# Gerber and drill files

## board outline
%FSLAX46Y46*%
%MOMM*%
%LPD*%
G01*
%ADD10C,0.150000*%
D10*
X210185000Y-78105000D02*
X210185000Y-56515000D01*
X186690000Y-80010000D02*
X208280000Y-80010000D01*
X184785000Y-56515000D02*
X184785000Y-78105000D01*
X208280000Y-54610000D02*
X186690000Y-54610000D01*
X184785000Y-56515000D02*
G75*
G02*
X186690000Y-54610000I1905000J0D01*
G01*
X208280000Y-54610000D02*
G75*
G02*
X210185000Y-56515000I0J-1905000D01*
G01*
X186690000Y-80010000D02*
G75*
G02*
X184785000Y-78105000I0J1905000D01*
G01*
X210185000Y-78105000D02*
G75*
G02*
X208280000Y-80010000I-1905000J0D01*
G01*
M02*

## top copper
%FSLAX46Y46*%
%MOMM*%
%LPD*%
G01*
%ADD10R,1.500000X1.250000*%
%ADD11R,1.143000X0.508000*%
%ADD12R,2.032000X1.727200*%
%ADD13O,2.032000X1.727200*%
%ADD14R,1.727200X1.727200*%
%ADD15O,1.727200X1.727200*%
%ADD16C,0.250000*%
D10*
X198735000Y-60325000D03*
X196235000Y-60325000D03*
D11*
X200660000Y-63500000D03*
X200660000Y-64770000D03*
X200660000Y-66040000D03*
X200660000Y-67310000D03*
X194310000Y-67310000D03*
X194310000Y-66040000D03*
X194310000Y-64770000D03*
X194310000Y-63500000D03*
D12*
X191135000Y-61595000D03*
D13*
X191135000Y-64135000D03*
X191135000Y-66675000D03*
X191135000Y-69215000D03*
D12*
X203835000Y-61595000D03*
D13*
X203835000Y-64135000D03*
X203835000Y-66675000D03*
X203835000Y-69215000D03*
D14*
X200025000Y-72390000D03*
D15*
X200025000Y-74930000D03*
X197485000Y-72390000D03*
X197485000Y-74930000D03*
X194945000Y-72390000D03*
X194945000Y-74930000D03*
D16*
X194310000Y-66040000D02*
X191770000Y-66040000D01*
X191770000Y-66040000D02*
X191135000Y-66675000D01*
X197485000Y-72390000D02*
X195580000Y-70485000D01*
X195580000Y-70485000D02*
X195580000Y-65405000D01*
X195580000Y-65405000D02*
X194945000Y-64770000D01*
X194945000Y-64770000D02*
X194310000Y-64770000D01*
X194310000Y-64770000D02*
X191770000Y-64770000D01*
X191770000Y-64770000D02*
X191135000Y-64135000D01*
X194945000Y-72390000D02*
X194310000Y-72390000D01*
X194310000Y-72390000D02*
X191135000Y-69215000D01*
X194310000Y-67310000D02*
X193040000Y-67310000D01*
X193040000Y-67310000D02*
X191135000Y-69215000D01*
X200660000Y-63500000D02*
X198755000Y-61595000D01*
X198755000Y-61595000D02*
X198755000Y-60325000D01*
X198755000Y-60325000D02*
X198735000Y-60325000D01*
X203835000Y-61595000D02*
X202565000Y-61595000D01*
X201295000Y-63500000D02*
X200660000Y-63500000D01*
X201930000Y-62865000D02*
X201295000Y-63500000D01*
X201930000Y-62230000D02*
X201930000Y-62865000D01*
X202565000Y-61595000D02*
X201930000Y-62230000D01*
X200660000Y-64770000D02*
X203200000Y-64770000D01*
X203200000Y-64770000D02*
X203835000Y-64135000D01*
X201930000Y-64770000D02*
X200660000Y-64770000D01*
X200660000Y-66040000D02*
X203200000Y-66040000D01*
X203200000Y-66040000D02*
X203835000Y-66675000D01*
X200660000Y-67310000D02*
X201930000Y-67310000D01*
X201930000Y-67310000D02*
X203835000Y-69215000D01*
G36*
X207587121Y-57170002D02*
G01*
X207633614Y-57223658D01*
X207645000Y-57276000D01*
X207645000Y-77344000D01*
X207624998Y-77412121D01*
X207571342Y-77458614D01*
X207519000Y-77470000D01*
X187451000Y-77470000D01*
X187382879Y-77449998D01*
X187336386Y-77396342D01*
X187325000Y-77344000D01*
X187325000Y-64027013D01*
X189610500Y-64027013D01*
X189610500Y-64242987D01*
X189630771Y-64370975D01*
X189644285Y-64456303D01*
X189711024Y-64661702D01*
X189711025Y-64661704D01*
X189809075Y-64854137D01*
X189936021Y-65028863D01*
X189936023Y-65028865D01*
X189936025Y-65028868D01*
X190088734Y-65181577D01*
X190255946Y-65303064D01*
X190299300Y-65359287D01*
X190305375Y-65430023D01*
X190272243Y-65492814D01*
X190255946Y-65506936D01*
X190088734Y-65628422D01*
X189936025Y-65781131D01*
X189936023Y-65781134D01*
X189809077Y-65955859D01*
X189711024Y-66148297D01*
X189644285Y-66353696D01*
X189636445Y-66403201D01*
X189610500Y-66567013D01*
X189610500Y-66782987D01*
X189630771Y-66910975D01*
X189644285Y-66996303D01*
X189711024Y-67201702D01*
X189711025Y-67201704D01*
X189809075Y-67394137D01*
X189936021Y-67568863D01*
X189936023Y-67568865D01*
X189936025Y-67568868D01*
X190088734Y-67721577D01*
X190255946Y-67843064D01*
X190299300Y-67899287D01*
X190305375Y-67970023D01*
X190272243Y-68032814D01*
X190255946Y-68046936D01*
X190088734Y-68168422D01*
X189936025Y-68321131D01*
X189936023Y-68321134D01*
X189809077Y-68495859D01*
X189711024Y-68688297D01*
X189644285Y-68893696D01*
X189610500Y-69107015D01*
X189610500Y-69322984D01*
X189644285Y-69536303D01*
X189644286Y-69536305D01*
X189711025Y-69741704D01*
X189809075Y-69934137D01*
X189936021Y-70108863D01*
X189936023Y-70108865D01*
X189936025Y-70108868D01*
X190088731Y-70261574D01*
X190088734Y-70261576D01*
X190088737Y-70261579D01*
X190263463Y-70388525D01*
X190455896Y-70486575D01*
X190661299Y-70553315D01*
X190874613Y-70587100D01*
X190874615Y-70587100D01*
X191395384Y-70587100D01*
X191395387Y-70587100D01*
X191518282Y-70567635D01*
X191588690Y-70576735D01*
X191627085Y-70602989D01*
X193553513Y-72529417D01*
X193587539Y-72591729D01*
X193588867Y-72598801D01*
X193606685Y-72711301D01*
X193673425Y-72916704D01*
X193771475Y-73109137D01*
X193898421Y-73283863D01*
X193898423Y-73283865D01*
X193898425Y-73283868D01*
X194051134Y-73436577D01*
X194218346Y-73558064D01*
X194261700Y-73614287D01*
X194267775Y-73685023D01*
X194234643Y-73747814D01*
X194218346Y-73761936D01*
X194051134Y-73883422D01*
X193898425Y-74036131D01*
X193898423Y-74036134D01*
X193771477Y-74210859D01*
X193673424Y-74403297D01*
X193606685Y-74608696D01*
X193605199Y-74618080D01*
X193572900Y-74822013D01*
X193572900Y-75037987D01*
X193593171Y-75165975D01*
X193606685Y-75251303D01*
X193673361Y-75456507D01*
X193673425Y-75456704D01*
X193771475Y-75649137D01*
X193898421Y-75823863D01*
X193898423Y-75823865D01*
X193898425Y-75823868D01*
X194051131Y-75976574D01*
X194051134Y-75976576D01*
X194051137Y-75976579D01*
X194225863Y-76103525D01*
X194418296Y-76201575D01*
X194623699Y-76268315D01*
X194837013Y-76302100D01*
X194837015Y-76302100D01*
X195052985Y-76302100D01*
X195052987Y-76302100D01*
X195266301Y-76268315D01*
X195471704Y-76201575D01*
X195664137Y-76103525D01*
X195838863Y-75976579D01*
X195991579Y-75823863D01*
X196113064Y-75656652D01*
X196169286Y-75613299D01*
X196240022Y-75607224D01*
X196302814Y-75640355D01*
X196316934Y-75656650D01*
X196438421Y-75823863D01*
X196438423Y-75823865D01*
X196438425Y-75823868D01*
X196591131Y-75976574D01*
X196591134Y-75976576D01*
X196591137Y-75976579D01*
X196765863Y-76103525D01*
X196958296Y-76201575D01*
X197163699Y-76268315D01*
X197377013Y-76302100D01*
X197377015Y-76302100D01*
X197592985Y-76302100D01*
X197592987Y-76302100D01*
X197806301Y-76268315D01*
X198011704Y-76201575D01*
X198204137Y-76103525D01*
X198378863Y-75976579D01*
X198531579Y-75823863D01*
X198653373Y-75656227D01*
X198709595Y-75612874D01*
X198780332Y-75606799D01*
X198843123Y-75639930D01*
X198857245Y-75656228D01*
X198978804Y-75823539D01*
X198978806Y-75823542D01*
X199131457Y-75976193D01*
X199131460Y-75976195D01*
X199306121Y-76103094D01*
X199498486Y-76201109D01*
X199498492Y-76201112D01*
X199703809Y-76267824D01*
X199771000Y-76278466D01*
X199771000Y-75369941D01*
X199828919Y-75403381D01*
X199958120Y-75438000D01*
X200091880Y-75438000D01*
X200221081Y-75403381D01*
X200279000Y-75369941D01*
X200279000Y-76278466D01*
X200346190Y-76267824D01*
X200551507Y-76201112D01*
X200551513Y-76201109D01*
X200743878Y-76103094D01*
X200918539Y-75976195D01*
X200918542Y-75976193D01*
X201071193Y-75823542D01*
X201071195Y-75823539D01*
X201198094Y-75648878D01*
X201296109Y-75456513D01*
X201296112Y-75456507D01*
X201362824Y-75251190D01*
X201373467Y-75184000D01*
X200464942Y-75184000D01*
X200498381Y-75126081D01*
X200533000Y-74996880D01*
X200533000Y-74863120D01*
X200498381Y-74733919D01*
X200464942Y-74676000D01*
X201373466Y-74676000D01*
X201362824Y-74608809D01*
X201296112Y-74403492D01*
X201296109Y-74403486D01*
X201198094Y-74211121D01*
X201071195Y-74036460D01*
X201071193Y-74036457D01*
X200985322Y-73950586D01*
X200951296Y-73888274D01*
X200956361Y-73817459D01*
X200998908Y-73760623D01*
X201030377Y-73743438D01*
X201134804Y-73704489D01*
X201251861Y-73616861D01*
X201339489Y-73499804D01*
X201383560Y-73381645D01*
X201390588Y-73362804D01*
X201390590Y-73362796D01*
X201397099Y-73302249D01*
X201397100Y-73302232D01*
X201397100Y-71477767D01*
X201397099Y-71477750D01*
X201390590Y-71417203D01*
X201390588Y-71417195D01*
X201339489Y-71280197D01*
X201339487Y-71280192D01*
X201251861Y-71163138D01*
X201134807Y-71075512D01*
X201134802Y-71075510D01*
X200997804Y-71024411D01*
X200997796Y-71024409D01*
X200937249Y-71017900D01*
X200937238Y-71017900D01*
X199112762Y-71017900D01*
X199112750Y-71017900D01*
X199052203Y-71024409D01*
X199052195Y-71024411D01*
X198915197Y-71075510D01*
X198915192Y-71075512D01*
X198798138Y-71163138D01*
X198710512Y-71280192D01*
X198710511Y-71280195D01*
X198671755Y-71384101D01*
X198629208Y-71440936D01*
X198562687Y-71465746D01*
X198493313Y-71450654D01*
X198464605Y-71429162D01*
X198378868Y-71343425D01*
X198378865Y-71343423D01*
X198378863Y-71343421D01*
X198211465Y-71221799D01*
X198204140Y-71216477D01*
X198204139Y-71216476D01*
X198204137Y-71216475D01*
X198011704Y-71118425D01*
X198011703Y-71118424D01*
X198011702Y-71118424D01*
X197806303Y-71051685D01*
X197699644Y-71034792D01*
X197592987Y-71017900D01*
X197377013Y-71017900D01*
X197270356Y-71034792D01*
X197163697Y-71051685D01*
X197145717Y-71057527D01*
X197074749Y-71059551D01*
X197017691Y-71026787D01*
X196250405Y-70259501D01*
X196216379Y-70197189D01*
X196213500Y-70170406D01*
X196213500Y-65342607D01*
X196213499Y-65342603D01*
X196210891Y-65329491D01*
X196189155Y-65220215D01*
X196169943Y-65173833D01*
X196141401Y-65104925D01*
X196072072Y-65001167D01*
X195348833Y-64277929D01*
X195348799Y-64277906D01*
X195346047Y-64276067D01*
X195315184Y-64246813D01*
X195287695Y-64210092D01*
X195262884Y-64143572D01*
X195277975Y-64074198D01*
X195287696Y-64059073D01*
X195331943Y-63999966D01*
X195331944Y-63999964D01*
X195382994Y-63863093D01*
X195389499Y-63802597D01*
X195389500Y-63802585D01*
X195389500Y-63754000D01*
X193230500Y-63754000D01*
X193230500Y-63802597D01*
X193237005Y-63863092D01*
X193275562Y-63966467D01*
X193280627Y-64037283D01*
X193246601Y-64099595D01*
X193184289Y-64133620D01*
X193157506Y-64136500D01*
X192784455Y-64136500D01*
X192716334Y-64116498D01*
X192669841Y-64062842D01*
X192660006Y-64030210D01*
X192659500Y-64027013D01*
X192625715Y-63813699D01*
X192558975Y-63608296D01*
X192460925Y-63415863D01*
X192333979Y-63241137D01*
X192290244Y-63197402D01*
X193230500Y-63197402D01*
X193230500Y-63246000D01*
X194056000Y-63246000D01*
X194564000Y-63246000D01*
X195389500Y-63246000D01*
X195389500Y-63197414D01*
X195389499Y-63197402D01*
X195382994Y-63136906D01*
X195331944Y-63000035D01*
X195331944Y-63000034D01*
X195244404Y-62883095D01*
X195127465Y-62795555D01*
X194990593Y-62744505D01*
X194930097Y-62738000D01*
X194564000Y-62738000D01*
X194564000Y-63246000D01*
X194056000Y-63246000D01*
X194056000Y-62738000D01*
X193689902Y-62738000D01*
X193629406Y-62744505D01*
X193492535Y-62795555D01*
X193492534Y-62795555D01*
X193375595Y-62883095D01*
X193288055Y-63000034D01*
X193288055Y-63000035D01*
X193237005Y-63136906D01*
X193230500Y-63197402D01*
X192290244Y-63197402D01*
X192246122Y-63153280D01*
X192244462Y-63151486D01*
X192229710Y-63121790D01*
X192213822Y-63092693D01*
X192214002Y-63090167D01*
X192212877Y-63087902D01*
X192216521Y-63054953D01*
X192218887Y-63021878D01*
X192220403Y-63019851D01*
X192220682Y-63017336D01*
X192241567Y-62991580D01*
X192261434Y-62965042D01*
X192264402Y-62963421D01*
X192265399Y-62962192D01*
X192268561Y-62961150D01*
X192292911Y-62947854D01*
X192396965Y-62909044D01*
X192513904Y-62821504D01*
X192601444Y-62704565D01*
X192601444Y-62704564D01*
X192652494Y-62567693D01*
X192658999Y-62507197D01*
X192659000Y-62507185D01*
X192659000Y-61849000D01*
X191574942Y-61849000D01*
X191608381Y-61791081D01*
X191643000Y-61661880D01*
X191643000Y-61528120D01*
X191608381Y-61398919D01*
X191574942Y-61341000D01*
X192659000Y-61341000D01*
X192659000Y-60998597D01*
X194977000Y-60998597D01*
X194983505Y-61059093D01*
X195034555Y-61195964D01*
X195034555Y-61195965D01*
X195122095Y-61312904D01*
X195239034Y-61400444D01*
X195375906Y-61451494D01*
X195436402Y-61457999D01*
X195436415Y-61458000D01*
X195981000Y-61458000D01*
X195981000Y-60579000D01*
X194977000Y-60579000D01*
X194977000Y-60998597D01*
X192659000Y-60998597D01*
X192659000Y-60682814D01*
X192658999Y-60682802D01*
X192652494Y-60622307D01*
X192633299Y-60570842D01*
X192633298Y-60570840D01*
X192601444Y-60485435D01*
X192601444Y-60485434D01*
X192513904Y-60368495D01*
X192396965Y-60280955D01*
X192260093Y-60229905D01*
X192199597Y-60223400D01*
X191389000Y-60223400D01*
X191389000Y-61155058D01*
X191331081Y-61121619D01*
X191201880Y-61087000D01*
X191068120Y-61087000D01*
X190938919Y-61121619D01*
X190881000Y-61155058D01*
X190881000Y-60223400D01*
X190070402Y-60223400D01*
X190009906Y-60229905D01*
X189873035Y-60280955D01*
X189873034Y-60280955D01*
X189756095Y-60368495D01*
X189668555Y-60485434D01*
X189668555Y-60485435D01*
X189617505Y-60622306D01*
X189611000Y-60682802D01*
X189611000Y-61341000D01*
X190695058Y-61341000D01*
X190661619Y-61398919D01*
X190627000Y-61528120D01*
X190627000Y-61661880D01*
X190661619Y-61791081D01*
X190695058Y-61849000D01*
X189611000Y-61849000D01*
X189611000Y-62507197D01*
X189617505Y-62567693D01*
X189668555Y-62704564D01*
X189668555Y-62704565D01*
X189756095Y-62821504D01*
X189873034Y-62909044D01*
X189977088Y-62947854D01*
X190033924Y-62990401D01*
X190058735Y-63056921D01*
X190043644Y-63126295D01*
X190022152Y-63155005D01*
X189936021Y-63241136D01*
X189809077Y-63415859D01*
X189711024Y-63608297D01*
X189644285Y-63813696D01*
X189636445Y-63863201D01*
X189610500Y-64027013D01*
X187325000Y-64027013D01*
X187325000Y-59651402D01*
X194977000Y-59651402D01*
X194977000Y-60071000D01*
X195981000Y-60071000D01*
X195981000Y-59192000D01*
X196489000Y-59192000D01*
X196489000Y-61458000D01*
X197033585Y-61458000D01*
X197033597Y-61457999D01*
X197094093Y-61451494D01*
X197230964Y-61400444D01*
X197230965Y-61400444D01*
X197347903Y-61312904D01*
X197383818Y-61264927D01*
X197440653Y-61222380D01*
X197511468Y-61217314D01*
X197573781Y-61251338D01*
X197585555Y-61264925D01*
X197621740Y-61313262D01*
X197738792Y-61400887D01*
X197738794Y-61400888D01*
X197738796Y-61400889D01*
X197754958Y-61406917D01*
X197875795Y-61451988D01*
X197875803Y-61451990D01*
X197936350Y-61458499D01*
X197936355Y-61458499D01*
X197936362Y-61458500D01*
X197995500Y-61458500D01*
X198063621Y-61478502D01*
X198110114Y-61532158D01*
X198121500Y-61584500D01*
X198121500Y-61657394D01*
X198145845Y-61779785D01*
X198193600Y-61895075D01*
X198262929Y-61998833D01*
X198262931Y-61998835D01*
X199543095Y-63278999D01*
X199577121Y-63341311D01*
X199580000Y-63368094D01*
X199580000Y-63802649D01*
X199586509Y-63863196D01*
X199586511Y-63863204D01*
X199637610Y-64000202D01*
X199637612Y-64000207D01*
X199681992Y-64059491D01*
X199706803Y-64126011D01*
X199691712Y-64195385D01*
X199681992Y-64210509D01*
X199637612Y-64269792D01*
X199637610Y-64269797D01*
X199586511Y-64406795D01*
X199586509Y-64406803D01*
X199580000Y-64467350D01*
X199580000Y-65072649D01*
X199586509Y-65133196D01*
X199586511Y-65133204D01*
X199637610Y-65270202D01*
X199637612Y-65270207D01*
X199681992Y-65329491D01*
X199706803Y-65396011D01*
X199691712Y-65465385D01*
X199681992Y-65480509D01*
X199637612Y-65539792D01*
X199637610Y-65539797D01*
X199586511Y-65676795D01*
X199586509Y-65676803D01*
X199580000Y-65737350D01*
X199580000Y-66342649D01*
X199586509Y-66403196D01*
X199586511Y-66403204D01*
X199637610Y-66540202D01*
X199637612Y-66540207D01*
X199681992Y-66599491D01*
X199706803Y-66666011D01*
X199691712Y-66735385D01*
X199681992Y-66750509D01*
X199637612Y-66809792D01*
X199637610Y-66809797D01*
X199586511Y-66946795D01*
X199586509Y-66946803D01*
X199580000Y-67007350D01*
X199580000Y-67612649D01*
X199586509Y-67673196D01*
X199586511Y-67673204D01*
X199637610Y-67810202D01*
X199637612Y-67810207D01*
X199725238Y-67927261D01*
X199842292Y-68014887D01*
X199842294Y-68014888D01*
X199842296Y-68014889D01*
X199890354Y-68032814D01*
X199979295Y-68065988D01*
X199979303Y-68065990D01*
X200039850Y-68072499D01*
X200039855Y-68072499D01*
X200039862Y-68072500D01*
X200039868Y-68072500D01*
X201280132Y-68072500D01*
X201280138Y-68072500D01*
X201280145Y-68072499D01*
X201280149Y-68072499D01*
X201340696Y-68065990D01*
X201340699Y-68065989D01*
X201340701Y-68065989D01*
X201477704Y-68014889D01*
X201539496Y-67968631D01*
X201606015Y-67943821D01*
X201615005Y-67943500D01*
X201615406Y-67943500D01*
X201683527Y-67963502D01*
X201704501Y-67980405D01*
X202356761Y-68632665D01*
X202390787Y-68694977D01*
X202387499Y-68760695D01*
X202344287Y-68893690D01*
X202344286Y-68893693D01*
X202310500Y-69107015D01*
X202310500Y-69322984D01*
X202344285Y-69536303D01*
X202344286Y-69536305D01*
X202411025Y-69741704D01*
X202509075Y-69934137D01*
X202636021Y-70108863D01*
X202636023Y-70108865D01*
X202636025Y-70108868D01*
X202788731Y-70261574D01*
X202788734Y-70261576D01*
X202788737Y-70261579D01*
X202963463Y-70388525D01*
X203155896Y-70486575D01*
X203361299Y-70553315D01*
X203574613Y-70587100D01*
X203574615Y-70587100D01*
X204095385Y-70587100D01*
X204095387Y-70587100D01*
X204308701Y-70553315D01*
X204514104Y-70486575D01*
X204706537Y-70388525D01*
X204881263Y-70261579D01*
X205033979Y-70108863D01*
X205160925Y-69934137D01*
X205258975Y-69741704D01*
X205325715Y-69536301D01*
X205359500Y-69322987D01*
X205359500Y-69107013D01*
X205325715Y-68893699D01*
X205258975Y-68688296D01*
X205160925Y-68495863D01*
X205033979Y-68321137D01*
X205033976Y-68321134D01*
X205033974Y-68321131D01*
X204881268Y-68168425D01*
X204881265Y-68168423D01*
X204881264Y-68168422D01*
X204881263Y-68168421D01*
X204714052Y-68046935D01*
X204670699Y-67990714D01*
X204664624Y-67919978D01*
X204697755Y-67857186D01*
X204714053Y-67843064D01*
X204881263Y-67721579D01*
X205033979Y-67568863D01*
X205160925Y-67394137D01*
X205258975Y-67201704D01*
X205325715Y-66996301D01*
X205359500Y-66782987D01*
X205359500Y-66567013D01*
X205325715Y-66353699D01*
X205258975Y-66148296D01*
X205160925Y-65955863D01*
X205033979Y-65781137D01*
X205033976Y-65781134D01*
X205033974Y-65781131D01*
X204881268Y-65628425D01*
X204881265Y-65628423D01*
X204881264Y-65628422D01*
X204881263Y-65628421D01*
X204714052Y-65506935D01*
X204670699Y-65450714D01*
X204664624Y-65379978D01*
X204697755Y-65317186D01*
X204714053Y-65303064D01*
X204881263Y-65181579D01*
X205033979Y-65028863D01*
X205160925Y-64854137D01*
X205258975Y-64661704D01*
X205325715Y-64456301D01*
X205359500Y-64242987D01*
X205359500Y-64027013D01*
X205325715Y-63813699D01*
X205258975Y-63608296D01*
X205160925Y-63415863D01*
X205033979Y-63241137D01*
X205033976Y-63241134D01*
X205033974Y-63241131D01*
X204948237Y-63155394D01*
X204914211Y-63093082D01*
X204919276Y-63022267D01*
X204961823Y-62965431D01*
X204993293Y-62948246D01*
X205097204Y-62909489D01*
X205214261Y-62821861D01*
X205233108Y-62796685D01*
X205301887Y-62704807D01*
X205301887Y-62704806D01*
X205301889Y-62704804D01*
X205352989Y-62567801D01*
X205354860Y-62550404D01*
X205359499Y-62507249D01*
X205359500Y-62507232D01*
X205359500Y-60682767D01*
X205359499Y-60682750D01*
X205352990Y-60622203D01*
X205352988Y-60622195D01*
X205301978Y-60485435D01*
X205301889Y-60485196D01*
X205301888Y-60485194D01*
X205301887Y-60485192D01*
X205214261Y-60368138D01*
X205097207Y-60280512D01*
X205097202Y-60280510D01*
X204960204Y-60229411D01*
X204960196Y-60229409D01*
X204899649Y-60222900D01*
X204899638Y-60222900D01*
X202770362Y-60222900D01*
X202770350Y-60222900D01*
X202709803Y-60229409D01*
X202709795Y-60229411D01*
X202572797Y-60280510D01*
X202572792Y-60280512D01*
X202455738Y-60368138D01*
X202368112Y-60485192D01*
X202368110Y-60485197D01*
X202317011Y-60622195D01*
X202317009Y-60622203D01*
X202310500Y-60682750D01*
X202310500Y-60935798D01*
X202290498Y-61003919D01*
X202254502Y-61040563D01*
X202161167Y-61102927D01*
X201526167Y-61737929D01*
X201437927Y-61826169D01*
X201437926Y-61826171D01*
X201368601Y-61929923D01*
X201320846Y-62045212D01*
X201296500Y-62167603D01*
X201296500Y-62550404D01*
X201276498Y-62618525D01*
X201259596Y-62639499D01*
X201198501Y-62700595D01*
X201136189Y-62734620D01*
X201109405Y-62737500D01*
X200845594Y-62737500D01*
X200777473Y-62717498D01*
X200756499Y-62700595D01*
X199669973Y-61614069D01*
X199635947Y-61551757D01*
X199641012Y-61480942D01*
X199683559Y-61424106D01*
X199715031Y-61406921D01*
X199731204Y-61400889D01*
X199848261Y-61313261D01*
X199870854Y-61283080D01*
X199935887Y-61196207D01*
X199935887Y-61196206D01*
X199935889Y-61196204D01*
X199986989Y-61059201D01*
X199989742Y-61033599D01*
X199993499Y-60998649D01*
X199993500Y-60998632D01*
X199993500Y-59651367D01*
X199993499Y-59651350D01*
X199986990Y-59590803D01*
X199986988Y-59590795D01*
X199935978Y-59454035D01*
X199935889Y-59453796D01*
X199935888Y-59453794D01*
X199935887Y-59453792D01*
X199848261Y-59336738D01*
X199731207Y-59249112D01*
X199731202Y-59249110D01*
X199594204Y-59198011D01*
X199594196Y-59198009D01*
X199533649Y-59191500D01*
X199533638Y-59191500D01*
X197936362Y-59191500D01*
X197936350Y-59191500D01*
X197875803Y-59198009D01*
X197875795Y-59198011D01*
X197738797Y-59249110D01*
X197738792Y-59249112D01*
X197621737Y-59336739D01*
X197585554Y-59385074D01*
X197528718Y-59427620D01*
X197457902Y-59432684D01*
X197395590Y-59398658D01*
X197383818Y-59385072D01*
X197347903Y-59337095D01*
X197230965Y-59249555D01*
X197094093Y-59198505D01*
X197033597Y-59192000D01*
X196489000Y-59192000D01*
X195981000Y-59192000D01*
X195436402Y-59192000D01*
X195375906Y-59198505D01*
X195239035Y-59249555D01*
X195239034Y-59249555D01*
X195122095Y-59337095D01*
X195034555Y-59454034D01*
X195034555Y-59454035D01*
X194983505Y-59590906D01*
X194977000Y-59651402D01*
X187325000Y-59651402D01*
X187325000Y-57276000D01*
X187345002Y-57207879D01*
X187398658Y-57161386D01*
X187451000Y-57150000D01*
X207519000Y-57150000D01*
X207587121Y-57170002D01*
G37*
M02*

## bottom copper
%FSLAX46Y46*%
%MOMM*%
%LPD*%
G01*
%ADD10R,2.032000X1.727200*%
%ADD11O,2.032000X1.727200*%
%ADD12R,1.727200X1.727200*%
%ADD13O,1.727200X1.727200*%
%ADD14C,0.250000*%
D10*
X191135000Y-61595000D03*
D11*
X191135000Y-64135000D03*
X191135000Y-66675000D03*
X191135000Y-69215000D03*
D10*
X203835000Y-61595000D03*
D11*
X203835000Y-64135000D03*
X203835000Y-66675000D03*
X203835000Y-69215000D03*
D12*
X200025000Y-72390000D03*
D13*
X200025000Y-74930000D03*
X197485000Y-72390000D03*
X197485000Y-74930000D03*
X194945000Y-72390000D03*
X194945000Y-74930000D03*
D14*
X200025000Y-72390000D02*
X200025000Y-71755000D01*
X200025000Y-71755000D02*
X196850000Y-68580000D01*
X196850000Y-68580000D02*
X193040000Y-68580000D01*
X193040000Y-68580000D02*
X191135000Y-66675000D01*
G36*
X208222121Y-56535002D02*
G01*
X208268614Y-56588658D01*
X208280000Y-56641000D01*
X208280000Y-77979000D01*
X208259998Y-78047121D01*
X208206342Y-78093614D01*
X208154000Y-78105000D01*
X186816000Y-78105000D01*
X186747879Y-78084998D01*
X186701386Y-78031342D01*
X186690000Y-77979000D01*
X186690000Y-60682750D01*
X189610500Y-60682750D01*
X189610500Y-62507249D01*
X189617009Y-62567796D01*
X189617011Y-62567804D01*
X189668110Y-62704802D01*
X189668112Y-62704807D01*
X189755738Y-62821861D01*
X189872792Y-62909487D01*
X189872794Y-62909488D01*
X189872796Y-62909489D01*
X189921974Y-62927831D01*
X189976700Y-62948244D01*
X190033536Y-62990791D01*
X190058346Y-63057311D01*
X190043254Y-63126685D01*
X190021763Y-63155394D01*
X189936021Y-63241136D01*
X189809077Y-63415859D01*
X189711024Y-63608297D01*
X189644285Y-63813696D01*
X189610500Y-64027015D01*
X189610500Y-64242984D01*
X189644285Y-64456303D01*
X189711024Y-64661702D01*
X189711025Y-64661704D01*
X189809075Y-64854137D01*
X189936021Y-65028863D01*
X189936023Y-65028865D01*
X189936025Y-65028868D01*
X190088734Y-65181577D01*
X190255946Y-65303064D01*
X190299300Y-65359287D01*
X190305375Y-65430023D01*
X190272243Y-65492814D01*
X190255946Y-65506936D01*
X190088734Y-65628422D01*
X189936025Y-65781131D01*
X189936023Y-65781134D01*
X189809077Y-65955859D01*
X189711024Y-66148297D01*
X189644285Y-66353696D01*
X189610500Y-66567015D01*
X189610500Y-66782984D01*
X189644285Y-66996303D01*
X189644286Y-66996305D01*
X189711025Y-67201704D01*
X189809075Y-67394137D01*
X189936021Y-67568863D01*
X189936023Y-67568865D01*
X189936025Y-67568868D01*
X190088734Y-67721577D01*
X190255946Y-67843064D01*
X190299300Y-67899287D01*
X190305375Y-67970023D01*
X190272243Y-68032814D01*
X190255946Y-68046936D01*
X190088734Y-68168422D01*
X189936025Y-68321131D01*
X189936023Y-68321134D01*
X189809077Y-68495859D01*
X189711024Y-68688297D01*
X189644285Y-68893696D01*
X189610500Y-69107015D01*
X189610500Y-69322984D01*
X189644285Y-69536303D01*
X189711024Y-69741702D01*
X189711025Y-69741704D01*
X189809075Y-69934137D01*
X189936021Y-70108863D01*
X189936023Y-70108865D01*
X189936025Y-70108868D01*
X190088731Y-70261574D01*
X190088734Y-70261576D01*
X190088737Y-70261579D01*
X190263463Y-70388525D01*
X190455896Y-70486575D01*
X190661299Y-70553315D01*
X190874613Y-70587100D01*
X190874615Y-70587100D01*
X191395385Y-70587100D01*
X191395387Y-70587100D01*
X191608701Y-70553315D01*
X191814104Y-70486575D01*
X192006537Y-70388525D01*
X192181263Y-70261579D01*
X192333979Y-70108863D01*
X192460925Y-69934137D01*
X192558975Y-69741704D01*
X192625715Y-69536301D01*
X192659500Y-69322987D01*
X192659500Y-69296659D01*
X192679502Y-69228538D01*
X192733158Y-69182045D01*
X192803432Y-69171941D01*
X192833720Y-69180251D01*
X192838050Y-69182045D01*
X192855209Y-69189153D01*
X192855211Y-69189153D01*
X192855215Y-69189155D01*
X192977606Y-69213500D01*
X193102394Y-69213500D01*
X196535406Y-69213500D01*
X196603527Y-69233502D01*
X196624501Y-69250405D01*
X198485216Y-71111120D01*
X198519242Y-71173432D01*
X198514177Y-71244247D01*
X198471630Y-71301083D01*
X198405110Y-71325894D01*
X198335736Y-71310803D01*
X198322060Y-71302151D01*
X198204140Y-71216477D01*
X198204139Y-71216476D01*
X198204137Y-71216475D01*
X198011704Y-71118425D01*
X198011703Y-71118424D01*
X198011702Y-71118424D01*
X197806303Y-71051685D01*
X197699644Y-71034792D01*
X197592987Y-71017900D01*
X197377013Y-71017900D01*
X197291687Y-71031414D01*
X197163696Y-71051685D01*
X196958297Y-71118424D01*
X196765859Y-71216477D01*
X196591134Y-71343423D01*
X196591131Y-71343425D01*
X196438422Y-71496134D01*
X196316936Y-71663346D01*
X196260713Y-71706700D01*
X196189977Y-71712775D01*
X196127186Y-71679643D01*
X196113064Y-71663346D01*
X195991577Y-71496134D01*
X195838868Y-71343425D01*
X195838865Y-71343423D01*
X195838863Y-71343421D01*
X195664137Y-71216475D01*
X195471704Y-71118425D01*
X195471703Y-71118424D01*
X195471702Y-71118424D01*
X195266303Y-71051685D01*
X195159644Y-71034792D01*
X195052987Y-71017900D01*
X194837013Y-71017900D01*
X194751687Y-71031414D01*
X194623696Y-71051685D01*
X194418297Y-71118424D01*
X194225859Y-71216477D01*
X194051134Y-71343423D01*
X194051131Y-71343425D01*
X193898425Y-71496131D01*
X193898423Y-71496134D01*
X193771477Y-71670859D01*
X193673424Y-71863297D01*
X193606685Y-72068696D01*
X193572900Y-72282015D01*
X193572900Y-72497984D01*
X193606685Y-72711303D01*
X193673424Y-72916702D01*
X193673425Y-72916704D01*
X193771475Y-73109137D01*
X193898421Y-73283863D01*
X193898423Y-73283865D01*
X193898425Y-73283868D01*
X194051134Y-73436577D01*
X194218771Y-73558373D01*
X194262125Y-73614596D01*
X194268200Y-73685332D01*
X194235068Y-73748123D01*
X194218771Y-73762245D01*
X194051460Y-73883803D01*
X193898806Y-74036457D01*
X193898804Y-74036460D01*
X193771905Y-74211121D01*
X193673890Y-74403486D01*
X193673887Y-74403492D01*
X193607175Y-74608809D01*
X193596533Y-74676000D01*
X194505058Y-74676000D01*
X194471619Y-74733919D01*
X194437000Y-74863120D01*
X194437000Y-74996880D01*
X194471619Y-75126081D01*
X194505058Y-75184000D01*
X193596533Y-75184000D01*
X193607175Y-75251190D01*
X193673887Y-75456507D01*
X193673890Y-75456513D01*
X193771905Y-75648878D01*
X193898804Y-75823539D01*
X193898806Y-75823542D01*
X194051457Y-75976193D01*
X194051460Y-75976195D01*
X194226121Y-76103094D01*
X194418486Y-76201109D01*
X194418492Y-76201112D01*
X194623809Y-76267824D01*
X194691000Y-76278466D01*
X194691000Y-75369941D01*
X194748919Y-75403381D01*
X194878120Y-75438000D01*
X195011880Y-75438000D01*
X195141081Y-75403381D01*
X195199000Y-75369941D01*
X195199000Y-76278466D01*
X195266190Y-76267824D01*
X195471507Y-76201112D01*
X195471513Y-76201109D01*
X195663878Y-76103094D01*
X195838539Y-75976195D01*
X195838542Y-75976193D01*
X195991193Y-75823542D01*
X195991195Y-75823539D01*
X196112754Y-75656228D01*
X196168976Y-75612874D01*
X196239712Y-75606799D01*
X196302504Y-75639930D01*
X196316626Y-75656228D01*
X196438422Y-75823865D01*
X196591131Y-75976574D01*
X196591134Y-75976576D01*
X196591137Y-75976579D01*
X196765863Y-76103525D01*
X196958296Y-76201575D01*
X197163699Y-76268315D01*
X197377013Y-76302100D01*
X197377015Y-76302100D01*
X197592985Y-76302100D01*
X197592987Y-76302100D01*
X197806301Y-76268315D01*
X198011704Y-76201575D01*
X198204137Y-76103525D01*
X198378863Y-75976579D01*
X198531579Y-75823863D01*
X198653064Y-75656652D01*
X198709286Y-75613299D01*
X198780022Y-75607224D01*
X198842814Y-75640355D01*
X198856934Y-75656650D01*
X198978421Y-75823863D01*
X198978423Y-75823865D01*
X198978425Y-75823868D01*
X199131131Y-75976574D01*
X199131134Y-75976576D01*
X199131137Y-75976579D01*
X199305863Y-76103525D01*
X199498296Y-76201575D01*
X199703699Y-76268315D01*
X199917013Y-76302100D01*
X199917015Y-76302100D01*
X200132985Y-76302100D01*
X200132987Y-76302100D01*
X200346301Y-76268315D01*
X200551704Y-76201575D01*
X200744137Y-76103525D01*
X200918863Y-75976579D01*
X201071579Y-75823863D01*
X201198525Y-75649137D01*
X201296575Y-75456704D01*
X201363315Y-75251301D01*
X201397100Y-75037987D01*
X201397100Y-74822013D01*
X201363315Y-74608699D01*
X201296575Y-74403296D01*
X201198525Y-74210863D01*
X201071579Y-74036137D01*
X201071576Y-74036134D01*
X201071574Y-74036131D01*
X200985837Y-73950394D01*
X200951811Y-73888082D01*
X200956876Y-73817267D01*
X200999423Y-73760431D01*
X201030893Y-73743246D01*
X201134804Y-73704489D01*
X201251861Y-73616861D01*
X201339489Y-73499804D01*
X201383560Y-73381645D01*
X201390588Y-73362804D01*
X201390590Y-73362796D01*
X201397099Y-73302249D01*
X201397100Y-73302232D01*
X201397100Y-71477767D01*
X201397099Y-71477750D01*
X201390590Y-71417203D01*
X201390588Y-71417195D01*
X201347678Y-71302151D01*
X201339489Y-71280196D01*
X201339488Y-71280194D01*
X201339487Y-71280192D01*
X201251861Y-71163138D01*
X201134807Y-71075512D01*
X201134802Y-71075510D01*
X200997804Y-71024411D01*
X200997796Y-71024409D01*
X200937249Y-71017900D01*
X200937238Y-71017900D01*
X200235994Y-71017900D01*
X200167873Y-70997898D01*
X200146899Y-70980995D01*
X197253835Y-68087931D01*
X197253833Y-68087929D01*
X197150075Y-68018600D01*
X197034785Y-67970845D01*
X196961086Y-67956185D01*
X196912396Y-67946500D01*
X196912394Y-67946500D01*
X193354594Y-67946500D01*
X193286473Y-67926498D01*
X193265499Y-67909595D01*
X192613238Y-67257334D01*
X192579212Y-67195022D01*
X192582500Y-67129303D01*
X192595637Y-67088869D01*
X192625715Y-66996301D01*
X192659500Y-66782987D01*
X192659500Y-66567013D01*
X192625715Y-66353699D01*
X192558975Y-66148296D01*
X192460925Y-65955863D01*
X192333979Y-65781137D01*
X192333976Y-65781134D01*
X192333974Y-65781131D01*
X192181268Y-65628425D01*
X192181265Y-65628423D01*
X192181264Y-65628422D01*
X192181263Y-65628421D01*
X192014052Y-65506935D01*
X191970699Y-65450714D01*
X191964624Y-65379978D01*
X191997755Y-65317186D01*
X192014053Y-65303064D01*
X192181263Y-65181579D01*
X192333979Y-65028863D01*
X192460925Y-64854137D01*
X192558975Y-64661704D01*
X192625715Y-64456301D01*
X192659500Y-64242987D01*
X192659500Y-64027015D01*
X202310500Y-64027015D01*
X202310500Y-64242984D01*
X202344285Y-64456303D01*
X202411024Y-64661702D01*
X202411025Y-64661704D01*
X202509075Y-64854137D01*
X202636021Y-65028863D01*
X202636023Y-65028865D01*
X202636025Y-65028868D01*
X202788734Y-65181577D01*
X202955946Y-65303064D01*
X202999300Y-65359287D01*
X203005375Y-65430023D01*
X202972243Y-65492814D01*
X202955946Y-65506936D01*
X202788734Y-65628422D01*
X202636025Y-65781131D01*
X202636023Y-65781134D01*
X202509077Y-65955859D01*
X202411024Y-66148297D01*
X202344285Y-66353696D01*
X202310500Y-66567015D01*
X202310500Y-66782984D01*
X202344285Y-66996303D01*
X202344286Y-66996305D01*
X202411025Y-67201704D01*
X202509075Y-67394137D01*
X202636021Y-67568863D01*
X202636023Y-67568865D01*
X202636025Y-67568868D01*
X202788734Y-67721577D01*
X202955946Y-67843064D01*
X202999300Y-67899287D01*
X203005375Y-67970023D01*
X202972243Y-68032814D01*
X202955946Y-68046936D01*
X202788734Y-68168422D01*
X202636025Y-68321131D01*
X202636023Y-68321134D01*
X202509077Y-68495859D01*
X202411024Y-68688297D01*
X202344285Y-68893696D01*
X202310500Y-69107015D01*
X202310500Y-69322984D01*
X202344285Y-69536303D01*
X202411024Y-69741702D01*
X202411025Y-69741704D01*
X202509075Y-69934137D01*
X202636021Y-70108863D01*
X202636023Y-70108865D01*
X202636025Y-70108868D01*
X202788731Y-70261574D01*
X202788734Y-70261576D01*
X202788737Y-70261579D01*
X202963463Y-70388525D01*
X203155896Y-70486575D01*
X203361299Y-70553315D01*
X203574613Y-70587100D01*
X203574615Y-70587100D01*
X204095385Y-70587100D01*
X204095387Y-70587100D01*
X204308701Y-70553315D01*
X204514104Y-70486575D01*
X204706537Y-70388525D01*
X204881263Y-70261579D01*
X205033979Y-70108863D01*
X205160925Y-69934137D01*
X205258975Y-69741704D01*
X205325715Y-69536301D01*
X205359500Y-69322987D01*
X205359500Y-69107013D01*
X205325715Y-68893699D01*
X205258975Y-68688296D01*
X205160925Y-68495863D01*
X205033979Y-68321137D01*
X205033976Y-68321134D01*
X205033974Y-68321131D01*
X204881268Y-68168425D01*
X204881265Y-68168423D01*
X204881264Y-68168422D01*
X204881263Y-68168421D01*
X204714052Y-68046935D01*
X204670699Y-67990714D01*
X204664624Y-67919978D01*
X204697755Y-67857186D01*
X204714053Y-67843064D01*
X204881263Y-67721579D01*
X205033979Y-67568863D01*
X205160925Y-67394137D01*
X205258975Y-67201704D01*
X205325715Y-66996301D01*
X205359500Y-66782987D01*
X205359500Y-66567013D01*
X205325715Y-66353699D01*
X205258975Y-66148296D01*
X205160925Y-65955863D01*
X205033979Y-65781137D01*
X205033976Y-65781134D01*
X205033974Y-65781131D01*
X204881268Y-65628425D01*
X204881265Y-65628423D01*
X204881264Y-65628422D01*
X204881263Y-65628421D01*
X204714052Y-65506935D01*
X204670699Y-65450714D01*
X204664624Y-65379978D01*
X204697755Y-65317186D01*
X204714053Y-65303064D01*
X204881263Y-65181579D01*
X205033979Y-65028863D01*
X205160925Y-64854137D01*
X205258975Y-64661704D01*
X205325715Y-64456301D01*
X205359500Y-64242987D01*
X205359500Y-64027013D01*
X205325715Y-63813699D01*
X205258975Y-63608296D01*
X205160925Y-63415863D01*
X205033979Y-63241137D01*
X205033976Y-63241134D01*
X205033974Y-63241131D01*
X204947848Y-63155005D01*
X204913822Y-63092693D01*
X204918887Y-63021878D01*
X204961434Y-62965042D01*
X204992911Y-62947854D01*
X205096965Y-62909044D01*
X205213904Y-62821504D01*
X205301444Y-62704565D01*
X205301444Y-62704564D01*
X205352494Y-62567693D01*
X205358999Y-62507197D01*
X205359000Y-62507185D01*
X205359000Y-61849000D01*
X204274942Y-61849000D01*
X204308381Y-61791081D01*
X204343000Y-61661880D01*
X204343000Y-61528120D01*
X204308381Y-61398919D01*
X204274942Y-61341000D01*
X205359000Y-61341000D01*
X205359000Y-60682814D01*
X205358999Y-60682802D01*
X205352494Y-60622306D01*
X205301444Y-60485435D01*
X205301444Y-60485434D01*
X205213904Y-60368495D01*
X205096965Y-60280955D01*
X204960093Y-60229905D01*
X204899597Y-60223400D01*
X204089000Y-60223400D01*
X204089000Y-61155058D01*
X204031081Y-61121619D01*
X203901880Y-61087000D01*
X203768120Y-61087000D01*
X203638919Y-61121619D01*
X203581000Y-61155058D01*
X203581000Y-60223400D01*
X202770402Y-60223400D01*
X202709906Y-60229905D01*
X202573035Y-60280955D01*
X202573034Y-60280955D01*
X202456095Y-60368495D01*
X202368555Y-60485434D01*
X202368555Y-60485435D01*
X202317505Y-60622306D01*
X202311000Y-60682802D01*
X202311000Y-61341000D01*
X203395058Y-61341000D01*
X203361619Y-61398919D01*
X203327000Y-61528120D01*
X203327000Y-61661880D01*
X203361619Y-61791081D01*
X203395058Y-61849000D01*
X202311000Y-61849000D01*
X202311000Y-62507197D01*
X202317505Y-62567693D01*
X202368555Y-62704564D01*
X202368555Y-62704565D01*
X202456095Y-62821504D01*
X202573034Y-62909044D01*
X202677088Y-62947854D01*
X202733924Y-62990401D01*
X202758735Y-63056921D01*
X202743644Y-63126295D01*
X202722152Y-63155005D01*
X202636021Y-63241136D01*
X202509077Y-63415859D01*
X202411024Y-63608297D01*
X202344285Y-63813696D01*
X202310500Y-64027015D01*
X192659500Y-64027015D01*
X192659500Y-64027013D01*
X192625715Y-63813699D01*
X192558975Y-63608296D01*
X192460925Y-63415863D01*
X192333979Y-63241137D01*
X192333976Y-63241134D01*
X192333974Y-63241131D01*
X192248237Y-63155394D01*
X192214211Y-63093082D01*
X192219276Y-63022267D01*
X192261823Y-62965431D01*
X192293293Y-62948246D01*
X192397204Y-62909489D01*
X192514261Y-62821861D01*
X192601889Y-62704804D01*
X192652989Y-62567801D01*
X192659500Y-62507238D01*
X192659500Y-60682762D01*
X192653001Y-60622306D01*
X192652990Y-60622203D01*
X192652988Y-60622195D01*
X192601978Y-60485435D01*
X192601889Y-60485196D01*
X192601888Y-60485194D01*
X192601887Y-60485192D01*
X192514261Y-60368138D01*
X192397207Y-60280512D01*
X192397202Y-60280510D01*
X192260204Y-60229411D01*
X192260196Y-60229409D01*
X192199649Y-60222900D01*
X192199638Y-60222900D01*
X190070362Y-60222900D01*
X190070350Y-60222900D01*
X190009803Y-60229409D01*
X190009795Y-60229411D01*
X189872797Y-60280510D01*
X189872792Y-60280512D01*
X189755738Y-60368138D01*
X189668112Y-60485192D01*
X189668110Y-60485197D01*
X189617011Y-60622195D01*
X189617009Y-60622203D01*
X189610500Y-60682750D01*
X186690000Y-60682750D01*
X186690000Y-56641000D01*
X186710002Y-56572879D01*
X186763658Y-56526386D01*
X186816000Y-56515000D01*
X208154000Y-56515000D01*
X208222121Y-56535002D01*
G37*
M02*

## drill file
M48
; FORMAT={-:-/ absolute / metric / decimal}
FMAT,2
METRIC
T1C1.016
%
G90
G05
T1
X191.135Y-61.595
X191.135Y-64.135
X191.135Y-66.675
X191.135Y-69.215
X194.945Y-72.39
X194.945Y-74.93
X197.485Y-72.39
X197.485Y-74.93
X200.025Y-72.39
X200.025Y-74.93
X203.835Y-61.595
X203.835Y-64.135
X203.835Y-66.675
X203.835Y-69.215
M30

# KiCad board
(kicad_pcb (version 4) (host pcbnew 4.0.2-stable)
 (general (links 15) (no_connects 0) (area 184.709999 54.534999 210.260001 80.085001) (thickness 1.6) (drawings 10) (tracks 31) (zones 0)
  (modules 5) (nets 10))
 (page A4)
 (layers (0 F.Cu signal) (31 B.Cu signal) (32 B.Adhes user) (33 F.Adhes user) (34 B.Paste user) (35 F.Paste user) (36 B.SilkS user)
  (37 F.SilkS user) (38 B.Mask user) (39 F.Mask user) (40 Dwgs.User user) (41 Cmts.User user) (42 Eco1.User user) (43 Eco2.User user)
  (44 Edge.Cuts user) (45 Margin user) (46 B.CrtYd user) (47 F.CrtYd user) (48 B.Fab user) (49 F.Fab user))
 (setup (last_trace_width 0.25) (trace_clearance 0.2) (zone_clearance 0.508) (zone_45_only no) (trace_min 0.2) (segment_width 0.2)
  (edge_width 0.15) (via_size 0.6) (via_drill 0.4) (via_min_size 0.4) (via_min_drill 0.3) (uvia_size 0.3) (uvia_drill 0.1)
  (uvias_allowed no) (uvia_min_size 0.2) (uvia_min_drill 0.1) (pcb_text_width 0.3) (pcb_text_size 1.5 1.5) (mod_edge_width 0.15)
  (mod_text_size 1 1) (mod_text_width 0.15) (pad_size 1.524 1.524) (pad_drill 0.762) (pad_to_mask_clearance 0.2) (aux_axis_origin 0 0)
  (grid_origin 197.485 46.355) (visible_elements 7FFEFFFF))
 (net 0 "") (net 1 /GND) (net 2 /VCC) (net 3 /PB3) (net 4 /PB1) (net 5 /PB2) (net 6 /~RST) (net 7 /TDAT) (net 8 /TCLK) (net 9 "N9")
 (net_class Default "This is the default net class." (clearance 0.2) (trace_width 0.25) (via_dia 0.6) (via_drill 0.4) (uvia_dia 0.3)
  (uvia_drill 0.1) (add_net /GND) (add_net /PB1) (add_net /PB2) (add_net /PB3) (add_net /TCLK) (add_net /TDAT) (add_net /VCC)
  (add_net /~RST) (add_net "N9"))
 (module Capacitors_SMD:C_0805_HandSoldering (layer F.Cu) (at 197.485 60.325 180)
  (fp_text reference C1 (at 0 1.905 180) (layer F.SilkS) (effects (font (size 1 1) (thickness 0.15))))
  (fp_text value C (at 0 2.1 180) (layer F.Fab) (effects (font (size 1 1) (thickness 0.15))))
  (pad 1 smd rect (at -1.25 0 180) (size 1.5 1.25) (layers F.Cu F.Paste F.Mask) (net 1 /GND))
  (pad 2 smd rect (at 1.25 0 180) (size 1.5 1.25) (layers F.Cu F.Paste F.Mask) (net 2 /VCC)))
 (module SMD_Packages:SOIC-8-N (layer F.Cu) (at 197.485 65.405 270)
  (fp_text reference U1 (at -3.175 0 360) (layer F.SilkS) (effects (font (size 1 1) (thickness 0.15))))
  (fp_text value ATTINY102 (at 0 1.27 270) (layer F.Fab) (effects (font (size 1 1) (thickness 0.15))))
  (pad 8 smd rect (at -1.905 -3.175 270) (size 0.508 1.143) (layers F.Cu F.Paste F.Mask) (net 1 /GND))
  (pad 7 smd rect (at -0.635 -3.175 270) (size 0.508 1.143) (layers F.Cu F.Paste F.Mask) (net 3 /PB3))
  (pad 6 smd rect (at 0.635 -3.175 270) (size 0.508 1.143) (layers F.Cu F.Paste F.Mask) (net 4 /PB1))
  (pad 5 smd rect (at 1.905 -3.175 270) (size 0.508 1.143) (layers F.Cu F.Paste F.Mask) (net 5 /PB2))
  (pad 4 smd rect (at 1.905 3.175 270) (size 0.508 1.143) (layers F.Cu F.Paste F.Mask) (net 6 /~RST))
  (pad 3 smd rect (at 0.635 3.175 270) (size 0.508 1.143) (layers F.Cu F.Paste F.Mask) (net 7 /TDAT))
  (pad 2 smd rect (at -0.635 3.175 270) (size 0.508 1.143) (layers F.Cu F.Paste F.Mask) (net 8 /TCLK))
  (pad 1 smd rect (at -1.905 3.175 270) (size 0.508 1.143) (layers F.Cu F.Paste F.Mask) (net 2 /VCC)))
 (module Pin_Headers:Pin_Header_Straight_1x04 (layer F.Cu) (at 191.135 61.595)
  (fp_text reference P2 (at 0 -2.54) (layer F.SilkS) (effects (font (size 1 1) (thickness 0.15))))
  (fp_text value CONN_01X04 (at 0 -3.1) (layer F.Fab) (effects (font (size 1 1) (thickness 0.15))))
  (pad 1 thru_hole rect (at 0 0) (size 2.032 1.7272) (drill 1.016) (layers *.Cu *.Mask F.SilkS) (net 2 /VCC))
  (pad 2 thru_hole oval (at 0 2.54) (size 2.032 1.7272) (drill 1.016) (layers *.Cu *.Mask F.SilkS) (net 8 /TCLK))
  (pad 3 thru_hole oval (at 0 5.08) (size 2.032 1.7272) (drill 1.016) (layers *.Cu *.Mask F.SilkS) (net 7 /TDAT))
  (pad 4 thru_hole oval (at 0 7.62) (size 2.032 1.7272) (drill 1.016) (layers *.Cu *.Mask F.SilkS) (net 6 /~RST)))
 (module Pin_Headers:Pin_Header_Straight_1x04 (layer F.Cu) (at 203.835 61.595)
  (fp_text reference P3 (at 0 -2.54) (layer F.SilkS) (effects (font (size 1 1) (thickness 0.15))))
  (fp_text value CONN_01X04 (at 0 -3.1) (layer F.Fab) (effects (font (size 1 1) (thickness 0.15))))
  (pad 1 thru_hole rect (at 0 0) (size 2.032 1.7272) (drill 1.016) (layers *.Cu *.Mask F.SilkS) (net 1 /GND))
  (pad 2 thru_hole oval (at 0 2.54) (size 2.032 1.7272) (drill 1.016) (layers *.Cu *.Mask F.SilkS) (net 3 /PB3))
  (pad 3 thru_hole oval (at 0 5.08) (size 2.032 1.7272) (drill 1.016) (layers *.Cu *.Mask F.SilkS) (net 4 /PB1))
  (pad 4 thru_hole oval (at 0 7.62) (size 2.032 1.7272) (drill 1.016) (layers *.Cu *.Mask F.SilkS) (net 5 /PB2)))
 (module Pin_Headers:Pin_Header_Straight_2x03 (layer F.Cu) (at 200.025 72.39 270)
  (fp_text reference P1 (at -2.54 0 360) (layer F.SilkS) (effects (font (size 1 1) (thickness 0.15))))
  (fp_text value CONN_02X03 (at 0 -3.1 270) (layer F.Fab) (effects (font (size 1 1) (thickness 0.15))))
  (pad 1 thru_hole rect (at 0 0 270) (size 1.7272 1.7272) (drill 1.016) (layers *.Cu *.Mask F.SilkS) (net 7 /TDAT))
  (pad 2 thru_hole oval (at 2.54 0 270) (size 1.7272 1.7272) (drill 1.016) (layers *.Cu *.Mask F.SilkS) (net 2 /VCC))
  (pad 3 thru_hole oval (at 0 2.54 270) (size 1.7272 1.7272) (drill 1.016) (layers *.Cu *.Mask F.SilkS) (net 8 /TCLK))
  (pad 4 thru_hole oval (at 2.54 2.54 270) (size 1.7272 1.7272) (drill 1.016) (layers *.Cu *.Mask F.SilkS) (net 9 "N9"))
  (pad 5 thru_hole oval (at 0 5.08 270) (size 1.7272 1.7272) (drill 1.016) (layers *.Cu *.Mask F.SilkS) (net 6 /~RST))
  (pad 6 thru_hole oval (at 2.54 5.08 270) (size 1.7272 1.7272) (drill 1.016) (layers *.Cu *.Mask F.SilkS) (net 1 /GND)))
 (gr_line (start 210.185 78.105) (end 210.185 56.515) (angle 90) (layer Edge.Cuts) (width 0.15))
 (gr_line (start 186.69 80.01) (end 208.28 80.01) (angle 90) (layer Edge.Cuts) (width 0.15))
 (gr_line (start 184.785 56.515) (end 184.785 78.105) (angle 90) (layer Edge.Cuts) (width 0.15))
 (gr_line (start 208.28 54.61) (end 186.69 54.61) (angle 90) (layer Edge.Cuts) (width 0.15))
 (gr_arc (start 186.69 56.515) (end 184.785 56.515) (angle 90) (layer Edge.Cuts) (width 0.15))
 (gr_arc (start 208.28 56.515) (end 208.28 54.61) (angle 90) (layer Edge.Cuts) (width 0.15))
 (gr_arc (start 186.69 78.105) (end 186.69 80.01) (angle 90) (layer Edge.Cuts) (width 0.15))
 (gr_arc (start 208.28 78.105) (end 210.185 78.105) (angle 90) (layer Edge.Cuts) (width 0.15))
 (segment (start 200.025 72.39) (end 200.025 71.755) (width 0.25) (layer B.Cu) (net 7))
 (segment (start 200.025 71.755) (end 196.85 68.58) (width 0.25) (layer B.Cu) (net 7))
 (segment (start 196.85 68.58) (end 193.04 68.58) (width 0.25) (layer B.Cu) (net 7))
 (segment (start 193.04 68.58) (end 191.135 66.675) (width 0.25) (layer B.Cu) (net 7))
 (segment (start 194.31 66.04) (end 191.77 66.04) (width 0.25) (layer F.Cu) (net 7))
 (segment (start 191.77 66.04) (end 191.135 66.675) (width 0.25) (layer F.Cu) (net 7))
 (segment (start 197.485 72.39) (end 195.58 70.485) (width 0.25) (layer F.Cu) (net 8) (status 80000))
 (segment (start 195.58 70.485) (end 195.58 65.405) (width 0.25) (layer F.Cu) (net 8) (status 80000))
 (segment (start 195.58 65.405) (end 194.945 64.77) (width 0.25) (layer F.Cu) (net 8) (status 80000))
 (segment (start 194.945 64.77) (end 194.31 64.77) (width 0.25) (layer F.Cu) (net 8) (status 80000))
 (segment (start 194.31 64.77) (end 191.77 64.77) (width 0.25) (layer F.Cu) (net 8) (status 80000))
 (segment (start 191.77 64.77) (end 191.135 64.135) (width 0.25) (layer F.Cu) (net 8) (status 80000))
 (segment (start 194.945 72.39) (end 194.31 72.39) (width 0.25) (layer F.Cu) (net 6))
 (segment (start 194.31 72.39) (end 191.135 69.215) (width 0.25) (layer F.Cu) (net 6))
 (segment (start 194.31 67.31) (end 193.04 67.31) (width 0.25) (layer F.Cu) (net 6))
 (segment (start 193.04 67.31) (end 191.135 69.215) (width 0.25) (layer F.Cu) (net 6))
 (segment (start 200.66 63.5) (end 198.755 61.595) (width 0.25) (layer F.Cu) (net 1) (status 80000))
 (segment (start 198.755 61.595) (end 198.755 60.325) (width 0.25) (layer F.Cu) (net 1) (status 80000))
 (segment (start 198.755 60.325) (end 198.735 60.325) (width 0.25) (layer F.Cu) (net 1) (status 80000))
 (segment (start 203.835 61.595) (end 202.565 61.595) (width 0.25) (layer F.Cu) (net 1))
 (segment (start 201.295 63.5) (end 200.66 63.5) (width 0.25) (layer F.Cu) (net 1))
 (segment (start 201.93 62.865) (end 201.295 63.5) (width 0.25) (layer F.Cu) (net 1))
 (segment (start 201.93 62.23) (end 201.93 62.865) (width 0.25) (layer F.Cu) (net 1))
 (segment (start 202.565 61.595) (end 201.93 62.23) (width 0.25) (layer F.Cu) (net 1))
 (segment (start 200.66 64.77) (end 203.2 64.77) (width 0.25) (layer F.Cu) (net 3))
 (segment (start 203.2 64.77) (end 203.835 64.135) (width 0.25) (layer F.Cu) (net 3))
 (segment (start 201.93 64.77) (end 200.66 64.77) (width 0.25) (layer F.Cu) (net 3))
 (segment (start 200.66 66.04) (end 203.2 66.04) (width 0.25) (layer F.Cu) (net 4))
 (segment (start 203.2 66.04) (end 203.835 66.675) (width 0.25) (layer F.Cu) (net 4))
 (segment (start 200.66 67.31) (end 201.93 67.31) (width 0.25) (layer F.Cu) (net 5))
 (segment (start 201.93 67.31) (end 203.835 69.215) (width 0.25) (layer F.Cu) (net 5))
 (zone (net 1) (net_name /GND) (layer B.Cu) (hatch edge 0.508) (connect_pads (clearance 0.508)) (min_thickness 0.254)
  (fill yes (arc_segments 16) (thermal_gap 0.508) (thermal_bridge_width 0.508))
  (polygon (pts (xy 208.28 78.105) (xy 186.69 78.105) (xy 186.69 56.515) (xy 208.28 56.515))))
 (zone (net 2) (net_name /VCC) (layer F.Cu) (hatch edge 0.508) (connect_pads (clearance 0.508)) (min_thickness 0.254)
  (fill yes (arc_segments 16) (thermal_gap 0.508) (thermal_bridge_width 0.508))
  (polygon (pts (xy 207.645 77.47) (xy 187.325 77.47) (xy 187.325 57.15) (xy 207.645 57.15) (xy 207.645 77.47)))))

